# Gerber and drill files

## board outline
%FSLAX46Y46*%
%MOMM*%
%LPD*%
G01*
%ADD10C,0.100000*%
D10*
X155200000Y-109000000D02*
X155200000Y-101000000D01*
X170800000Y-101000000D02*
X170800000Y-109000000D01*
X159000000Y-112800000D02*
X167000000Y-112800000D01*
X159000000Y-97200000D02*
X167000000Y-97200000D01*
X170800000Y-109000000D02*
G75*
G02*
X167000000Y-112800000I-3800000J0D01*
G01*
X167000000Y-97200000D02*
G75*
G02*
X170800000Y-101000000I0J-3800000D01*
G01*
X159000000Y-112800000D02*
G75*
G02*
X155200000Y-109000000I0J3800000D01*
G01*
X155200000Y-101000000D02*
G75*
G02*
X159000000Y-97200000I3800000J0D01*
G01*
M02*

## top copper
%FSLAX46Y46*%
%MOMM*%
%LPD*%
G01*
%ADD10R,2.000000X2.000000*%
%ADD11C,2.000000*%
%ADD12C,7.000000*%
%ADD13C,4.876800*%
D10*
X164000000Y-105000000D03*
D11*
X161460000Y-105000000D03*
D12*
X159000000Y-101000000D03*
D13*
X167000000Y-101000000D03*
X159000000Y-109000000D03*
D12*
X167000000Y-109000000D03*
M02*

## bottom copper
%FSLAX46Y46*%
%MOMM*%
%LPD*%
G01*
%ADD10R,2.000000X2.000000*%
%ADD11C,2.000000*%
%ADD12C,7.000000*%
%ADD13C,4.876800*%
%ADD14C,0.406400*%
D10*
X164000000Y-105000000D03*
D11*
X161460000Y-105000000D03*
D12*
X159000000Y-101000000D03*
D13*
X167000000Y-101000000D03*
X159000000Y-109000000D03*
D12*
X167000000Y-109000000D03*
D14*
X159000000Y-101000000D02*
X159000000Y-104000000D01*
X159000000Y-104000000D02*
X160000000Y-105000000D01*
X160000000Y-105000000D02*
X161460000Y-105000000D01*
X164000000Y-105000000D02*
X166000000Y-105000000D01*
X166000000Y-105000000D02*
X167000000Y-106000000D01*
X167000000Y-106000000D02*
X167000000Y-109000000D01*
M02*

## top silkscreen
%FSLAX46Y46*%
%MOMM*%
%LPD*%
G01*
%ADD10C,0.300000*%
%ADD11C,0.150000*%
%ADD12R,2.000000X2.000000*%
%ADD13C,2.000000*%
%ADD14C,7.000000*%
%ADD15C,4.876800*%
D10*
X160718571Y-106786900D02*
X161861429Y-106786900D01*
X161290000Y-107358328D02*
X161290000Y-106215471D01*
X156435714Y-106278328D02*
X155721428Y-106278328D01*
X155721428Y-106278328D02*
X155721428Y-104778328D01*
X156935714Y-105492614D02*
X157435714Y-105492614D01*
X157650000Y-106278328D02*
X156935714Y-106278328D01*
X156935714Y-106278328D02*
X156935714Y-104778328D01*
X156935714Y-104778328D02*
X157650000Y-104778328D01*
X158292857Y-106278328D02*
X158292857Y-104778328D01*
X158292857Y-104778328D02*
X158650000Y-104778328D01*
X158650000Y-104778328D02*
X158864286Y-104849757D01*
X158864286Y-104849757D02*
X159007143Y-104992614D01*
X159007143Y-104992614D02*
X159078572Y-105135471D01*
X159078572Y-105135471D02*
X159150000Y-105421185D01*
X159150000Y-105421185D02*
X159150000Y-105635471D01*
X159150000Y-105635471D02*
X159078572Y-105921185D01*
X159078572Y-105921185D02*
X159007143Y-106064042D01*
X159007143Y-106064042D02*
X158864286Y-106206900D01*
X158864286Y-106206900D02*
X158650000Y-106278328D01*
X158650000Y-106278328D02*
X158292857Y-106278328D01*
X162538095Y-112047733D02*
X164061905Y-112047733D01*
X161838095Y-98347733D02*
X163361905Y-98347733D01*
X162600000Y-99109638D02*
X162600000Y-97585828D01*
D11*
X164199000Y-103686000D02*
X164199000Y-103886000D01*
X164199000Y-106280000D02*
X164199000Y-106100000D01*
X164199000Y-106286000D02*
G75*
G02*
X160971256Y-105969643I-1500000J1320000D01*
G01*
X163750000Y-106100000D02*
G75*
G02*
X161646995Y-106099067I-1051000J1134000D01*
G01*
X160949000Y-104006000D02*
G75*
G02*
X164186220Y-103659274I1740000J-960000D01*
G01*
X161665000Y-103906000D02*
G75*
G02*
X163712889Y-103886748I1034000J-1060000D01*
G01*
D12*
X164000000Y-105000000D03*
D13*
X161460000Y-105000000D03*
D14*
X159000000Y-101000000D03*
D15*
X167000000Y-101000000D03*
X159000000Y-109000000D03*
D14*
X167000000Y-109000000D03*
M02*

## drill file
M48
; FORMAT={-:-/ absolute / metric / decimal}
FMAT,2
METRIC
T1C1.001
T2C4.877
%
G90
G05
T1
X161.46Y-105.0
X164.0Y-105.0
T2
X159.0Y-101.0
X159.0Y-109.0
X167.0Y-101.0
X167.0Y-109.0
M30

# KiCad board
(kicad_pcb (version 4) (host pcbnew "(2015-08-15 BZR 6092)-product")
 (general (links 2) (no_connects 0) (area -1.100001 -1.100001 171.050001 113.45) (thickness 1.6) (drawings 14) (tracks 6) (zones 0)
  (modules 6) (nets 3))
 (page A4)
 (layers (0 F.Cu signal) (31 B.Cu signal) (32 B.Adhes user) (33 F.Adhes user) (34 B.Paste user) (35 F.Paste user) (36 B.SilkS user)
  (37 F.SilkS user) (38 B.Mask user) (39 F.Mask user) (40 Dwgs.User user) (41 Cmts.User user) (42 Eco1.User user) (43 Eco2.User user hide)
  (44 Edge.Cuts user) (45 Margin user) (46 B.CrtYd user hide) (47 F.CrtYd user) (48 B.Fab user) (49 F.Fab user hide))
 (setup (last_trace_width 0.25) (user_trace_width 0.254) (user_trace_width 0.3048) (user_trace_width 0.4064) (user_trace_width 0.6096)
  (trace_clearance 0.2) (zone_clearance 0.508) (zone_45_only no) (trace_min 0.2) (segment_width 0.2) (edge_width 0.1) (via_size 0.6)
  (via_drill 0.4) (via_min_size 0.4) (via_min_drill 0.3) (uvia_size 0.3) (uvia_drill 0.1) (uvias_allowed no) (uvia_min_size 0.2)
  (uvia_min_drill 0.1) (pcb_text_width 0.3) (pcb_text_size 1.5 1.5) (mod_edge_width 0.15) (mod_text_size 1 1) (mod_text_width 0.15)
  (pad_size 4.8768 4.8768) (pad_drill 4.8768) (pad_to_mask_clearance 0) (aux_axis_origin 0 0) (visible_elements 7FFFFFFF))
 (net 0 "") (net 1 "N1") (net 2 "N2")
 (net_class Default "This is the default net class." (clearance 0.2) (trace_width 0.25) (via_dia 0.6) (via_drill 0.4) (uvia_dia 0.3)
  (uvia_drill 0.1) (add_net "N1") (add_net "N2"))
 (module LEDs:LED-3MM (layer F.Cu) (at 164 105 180)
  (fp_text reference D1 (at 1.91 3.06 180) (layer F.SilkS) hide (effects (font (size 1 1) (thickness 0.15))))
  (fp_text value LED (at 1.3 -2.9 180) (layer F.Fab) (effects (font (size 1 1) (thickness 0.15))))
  (fp_line (start -0.199 1.314) (end -0.199 1.114) (layer F.SilkS) (width 0.15))
  (fp_line (start -0.199 -1.28) (end -0.199 -1.1) (layer F.SilkS) (width 0.15))
  (fp_arc (start 1.301 0.034) (end -0.199 -1.286) (angle 108.5) (layer F.SilkS) (width 0.15))
  (fp_arc (start 1.301 0.034) (end 0.25 -1.1) (angle 85.7) (layer F.SilkS) (width 0.15))
  (fp_arc (start 1.311 0.034) (end 3.051 0.994) (angle 110) (layer F.SilkS) (width 0.15))
  (fp_arc (start 1.301 0.034) (end 2.335 1.094) (angle 87.5) (layer F.SilkS) (width 0.15))
  (pad 1 thru_hole rect (at 0 0 270) (size 2 2) (drill 1.00076) (layers *.Cu *.Mask F.SilkS) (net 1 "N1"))
  (pad 2 thru_hole circle (at 2.54 0 180) (size 2 2) (drill 1.00076) (layers *.Cu *.Mask F.SilkS) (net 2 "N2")))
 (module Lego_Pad (layer F.Cu) (at 159 101)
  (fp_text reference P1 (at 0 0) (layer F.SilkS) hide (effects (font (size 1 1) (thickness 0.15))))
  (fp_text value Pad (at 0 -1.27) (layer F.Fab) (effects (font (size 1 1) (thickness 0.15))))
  (pad 1 thru_hole circle (at 0 0) (size 7 7) (drill 4.8768) (layers *.Cu *.Mask F.SilkS) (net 2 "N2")))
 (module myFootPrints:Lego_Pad (layer F.Cu) (at 167 101)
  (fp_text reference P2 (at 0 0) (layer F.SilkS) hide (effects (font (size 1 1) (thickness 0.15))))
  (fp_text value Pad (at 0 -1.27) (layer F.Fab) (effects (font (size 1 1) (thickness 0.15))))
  (pad 1 thru_hole circle (at 0 0) (size 4.8768 4.8768) (drill 4.8768) (layers *.Cu *.Mask F.SilkS)))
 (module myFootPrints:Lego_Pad (layer F.Cu) (at 159 109)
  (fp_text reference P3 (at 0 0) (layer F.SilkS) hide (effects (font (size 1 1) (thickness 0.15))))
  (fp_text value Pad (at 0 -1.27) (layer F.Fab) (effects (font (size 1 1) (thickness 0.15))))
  (pad 1 thru_hole circle (at 0 0) (size 4.8768 4.8768) (drill 4.8768) (layers *.Cu *.Mask F.SilkS)))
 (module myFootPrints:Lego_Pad (layer F.Cu) (at 167 109)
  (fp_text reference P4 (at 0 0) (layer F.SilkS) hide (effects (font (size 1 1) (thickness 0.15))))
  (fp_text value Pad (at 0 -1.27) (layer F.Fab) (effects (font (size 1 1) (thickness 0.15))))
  (pad 1 thru_hole circle (at 0 0) (size 7 7) (drill 4.8768) (layers *.Cu *.Mask F.SilkS) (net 1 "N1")))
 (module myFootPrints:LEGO (layer F.Cu) (at 163 105)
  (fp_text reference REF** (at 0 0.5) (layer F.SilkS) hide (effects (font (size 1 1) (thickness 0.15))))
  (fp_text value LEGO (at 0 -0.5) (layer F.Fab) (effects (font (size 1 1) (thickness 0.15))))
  (fp_line (start -7.8 4) (end -7.8 -4) (layer Edge.Cuts) (width 0.1))
  (fp_line (start 7.8 -4) (end 7.8 4) (layer Edge.Cuts) (width 0.1))
  (fp_line (start -4 7.8) (end 4 7.8) (layer Edge.Cuts) (width 0.1))
  (fp_line (start -4 -7.8) (end 4 -7.8) (layer Edge.Cuts) (width 0.1))
  (fp_arc (start 4 4) (end 7.8 4) (angle 90) (layer Edge.Cuts) (width 0.1))
  (fp_arc (start 4 -4) (end 4 -7.8) (angle 90) (layer Edge.Cuts) (width 0.1))
  (fp_arc (start -4 4) (end -4 7.8) (angle 90) (layer Edge.Cuts) (width 0.1))
  (fp_arc (start -4 -4) (end -7.8 -4) (angle 90) (layer Edge.Cuts) (width 0.1)))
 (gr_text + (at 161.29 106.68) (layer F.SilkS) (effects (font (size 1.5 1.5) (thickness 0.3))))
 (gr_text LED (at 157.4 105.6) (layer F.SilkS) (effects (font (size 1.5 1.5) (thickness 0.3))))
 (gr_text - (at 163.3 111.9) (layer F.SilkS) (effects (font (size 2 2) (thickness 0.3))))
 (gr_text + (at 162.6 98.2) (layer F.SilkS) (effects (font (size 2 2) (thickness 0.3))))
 (segment (start 159 101) (end 159 104) (width 0.4064) (layer B.Cu) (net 2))
 (segment (start 159 104) (end 160 105) (width 0.4064) (layer B.Cu) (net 2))
 (segment (start 160 105) (end 161.46 105) (width 0.4064) (layer B.Cu) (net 2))
 (segment (start 164 105) (end 166 105) (width 0.4064) (layer B.Cu) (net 1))
 (segment (start 166 105) (end 167 106) (width 0.4064) (layer B.Cu) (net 1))
 (segment (start 167 106) (end 167 109) (width 0.4064) (layer B.Cu) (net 1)))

